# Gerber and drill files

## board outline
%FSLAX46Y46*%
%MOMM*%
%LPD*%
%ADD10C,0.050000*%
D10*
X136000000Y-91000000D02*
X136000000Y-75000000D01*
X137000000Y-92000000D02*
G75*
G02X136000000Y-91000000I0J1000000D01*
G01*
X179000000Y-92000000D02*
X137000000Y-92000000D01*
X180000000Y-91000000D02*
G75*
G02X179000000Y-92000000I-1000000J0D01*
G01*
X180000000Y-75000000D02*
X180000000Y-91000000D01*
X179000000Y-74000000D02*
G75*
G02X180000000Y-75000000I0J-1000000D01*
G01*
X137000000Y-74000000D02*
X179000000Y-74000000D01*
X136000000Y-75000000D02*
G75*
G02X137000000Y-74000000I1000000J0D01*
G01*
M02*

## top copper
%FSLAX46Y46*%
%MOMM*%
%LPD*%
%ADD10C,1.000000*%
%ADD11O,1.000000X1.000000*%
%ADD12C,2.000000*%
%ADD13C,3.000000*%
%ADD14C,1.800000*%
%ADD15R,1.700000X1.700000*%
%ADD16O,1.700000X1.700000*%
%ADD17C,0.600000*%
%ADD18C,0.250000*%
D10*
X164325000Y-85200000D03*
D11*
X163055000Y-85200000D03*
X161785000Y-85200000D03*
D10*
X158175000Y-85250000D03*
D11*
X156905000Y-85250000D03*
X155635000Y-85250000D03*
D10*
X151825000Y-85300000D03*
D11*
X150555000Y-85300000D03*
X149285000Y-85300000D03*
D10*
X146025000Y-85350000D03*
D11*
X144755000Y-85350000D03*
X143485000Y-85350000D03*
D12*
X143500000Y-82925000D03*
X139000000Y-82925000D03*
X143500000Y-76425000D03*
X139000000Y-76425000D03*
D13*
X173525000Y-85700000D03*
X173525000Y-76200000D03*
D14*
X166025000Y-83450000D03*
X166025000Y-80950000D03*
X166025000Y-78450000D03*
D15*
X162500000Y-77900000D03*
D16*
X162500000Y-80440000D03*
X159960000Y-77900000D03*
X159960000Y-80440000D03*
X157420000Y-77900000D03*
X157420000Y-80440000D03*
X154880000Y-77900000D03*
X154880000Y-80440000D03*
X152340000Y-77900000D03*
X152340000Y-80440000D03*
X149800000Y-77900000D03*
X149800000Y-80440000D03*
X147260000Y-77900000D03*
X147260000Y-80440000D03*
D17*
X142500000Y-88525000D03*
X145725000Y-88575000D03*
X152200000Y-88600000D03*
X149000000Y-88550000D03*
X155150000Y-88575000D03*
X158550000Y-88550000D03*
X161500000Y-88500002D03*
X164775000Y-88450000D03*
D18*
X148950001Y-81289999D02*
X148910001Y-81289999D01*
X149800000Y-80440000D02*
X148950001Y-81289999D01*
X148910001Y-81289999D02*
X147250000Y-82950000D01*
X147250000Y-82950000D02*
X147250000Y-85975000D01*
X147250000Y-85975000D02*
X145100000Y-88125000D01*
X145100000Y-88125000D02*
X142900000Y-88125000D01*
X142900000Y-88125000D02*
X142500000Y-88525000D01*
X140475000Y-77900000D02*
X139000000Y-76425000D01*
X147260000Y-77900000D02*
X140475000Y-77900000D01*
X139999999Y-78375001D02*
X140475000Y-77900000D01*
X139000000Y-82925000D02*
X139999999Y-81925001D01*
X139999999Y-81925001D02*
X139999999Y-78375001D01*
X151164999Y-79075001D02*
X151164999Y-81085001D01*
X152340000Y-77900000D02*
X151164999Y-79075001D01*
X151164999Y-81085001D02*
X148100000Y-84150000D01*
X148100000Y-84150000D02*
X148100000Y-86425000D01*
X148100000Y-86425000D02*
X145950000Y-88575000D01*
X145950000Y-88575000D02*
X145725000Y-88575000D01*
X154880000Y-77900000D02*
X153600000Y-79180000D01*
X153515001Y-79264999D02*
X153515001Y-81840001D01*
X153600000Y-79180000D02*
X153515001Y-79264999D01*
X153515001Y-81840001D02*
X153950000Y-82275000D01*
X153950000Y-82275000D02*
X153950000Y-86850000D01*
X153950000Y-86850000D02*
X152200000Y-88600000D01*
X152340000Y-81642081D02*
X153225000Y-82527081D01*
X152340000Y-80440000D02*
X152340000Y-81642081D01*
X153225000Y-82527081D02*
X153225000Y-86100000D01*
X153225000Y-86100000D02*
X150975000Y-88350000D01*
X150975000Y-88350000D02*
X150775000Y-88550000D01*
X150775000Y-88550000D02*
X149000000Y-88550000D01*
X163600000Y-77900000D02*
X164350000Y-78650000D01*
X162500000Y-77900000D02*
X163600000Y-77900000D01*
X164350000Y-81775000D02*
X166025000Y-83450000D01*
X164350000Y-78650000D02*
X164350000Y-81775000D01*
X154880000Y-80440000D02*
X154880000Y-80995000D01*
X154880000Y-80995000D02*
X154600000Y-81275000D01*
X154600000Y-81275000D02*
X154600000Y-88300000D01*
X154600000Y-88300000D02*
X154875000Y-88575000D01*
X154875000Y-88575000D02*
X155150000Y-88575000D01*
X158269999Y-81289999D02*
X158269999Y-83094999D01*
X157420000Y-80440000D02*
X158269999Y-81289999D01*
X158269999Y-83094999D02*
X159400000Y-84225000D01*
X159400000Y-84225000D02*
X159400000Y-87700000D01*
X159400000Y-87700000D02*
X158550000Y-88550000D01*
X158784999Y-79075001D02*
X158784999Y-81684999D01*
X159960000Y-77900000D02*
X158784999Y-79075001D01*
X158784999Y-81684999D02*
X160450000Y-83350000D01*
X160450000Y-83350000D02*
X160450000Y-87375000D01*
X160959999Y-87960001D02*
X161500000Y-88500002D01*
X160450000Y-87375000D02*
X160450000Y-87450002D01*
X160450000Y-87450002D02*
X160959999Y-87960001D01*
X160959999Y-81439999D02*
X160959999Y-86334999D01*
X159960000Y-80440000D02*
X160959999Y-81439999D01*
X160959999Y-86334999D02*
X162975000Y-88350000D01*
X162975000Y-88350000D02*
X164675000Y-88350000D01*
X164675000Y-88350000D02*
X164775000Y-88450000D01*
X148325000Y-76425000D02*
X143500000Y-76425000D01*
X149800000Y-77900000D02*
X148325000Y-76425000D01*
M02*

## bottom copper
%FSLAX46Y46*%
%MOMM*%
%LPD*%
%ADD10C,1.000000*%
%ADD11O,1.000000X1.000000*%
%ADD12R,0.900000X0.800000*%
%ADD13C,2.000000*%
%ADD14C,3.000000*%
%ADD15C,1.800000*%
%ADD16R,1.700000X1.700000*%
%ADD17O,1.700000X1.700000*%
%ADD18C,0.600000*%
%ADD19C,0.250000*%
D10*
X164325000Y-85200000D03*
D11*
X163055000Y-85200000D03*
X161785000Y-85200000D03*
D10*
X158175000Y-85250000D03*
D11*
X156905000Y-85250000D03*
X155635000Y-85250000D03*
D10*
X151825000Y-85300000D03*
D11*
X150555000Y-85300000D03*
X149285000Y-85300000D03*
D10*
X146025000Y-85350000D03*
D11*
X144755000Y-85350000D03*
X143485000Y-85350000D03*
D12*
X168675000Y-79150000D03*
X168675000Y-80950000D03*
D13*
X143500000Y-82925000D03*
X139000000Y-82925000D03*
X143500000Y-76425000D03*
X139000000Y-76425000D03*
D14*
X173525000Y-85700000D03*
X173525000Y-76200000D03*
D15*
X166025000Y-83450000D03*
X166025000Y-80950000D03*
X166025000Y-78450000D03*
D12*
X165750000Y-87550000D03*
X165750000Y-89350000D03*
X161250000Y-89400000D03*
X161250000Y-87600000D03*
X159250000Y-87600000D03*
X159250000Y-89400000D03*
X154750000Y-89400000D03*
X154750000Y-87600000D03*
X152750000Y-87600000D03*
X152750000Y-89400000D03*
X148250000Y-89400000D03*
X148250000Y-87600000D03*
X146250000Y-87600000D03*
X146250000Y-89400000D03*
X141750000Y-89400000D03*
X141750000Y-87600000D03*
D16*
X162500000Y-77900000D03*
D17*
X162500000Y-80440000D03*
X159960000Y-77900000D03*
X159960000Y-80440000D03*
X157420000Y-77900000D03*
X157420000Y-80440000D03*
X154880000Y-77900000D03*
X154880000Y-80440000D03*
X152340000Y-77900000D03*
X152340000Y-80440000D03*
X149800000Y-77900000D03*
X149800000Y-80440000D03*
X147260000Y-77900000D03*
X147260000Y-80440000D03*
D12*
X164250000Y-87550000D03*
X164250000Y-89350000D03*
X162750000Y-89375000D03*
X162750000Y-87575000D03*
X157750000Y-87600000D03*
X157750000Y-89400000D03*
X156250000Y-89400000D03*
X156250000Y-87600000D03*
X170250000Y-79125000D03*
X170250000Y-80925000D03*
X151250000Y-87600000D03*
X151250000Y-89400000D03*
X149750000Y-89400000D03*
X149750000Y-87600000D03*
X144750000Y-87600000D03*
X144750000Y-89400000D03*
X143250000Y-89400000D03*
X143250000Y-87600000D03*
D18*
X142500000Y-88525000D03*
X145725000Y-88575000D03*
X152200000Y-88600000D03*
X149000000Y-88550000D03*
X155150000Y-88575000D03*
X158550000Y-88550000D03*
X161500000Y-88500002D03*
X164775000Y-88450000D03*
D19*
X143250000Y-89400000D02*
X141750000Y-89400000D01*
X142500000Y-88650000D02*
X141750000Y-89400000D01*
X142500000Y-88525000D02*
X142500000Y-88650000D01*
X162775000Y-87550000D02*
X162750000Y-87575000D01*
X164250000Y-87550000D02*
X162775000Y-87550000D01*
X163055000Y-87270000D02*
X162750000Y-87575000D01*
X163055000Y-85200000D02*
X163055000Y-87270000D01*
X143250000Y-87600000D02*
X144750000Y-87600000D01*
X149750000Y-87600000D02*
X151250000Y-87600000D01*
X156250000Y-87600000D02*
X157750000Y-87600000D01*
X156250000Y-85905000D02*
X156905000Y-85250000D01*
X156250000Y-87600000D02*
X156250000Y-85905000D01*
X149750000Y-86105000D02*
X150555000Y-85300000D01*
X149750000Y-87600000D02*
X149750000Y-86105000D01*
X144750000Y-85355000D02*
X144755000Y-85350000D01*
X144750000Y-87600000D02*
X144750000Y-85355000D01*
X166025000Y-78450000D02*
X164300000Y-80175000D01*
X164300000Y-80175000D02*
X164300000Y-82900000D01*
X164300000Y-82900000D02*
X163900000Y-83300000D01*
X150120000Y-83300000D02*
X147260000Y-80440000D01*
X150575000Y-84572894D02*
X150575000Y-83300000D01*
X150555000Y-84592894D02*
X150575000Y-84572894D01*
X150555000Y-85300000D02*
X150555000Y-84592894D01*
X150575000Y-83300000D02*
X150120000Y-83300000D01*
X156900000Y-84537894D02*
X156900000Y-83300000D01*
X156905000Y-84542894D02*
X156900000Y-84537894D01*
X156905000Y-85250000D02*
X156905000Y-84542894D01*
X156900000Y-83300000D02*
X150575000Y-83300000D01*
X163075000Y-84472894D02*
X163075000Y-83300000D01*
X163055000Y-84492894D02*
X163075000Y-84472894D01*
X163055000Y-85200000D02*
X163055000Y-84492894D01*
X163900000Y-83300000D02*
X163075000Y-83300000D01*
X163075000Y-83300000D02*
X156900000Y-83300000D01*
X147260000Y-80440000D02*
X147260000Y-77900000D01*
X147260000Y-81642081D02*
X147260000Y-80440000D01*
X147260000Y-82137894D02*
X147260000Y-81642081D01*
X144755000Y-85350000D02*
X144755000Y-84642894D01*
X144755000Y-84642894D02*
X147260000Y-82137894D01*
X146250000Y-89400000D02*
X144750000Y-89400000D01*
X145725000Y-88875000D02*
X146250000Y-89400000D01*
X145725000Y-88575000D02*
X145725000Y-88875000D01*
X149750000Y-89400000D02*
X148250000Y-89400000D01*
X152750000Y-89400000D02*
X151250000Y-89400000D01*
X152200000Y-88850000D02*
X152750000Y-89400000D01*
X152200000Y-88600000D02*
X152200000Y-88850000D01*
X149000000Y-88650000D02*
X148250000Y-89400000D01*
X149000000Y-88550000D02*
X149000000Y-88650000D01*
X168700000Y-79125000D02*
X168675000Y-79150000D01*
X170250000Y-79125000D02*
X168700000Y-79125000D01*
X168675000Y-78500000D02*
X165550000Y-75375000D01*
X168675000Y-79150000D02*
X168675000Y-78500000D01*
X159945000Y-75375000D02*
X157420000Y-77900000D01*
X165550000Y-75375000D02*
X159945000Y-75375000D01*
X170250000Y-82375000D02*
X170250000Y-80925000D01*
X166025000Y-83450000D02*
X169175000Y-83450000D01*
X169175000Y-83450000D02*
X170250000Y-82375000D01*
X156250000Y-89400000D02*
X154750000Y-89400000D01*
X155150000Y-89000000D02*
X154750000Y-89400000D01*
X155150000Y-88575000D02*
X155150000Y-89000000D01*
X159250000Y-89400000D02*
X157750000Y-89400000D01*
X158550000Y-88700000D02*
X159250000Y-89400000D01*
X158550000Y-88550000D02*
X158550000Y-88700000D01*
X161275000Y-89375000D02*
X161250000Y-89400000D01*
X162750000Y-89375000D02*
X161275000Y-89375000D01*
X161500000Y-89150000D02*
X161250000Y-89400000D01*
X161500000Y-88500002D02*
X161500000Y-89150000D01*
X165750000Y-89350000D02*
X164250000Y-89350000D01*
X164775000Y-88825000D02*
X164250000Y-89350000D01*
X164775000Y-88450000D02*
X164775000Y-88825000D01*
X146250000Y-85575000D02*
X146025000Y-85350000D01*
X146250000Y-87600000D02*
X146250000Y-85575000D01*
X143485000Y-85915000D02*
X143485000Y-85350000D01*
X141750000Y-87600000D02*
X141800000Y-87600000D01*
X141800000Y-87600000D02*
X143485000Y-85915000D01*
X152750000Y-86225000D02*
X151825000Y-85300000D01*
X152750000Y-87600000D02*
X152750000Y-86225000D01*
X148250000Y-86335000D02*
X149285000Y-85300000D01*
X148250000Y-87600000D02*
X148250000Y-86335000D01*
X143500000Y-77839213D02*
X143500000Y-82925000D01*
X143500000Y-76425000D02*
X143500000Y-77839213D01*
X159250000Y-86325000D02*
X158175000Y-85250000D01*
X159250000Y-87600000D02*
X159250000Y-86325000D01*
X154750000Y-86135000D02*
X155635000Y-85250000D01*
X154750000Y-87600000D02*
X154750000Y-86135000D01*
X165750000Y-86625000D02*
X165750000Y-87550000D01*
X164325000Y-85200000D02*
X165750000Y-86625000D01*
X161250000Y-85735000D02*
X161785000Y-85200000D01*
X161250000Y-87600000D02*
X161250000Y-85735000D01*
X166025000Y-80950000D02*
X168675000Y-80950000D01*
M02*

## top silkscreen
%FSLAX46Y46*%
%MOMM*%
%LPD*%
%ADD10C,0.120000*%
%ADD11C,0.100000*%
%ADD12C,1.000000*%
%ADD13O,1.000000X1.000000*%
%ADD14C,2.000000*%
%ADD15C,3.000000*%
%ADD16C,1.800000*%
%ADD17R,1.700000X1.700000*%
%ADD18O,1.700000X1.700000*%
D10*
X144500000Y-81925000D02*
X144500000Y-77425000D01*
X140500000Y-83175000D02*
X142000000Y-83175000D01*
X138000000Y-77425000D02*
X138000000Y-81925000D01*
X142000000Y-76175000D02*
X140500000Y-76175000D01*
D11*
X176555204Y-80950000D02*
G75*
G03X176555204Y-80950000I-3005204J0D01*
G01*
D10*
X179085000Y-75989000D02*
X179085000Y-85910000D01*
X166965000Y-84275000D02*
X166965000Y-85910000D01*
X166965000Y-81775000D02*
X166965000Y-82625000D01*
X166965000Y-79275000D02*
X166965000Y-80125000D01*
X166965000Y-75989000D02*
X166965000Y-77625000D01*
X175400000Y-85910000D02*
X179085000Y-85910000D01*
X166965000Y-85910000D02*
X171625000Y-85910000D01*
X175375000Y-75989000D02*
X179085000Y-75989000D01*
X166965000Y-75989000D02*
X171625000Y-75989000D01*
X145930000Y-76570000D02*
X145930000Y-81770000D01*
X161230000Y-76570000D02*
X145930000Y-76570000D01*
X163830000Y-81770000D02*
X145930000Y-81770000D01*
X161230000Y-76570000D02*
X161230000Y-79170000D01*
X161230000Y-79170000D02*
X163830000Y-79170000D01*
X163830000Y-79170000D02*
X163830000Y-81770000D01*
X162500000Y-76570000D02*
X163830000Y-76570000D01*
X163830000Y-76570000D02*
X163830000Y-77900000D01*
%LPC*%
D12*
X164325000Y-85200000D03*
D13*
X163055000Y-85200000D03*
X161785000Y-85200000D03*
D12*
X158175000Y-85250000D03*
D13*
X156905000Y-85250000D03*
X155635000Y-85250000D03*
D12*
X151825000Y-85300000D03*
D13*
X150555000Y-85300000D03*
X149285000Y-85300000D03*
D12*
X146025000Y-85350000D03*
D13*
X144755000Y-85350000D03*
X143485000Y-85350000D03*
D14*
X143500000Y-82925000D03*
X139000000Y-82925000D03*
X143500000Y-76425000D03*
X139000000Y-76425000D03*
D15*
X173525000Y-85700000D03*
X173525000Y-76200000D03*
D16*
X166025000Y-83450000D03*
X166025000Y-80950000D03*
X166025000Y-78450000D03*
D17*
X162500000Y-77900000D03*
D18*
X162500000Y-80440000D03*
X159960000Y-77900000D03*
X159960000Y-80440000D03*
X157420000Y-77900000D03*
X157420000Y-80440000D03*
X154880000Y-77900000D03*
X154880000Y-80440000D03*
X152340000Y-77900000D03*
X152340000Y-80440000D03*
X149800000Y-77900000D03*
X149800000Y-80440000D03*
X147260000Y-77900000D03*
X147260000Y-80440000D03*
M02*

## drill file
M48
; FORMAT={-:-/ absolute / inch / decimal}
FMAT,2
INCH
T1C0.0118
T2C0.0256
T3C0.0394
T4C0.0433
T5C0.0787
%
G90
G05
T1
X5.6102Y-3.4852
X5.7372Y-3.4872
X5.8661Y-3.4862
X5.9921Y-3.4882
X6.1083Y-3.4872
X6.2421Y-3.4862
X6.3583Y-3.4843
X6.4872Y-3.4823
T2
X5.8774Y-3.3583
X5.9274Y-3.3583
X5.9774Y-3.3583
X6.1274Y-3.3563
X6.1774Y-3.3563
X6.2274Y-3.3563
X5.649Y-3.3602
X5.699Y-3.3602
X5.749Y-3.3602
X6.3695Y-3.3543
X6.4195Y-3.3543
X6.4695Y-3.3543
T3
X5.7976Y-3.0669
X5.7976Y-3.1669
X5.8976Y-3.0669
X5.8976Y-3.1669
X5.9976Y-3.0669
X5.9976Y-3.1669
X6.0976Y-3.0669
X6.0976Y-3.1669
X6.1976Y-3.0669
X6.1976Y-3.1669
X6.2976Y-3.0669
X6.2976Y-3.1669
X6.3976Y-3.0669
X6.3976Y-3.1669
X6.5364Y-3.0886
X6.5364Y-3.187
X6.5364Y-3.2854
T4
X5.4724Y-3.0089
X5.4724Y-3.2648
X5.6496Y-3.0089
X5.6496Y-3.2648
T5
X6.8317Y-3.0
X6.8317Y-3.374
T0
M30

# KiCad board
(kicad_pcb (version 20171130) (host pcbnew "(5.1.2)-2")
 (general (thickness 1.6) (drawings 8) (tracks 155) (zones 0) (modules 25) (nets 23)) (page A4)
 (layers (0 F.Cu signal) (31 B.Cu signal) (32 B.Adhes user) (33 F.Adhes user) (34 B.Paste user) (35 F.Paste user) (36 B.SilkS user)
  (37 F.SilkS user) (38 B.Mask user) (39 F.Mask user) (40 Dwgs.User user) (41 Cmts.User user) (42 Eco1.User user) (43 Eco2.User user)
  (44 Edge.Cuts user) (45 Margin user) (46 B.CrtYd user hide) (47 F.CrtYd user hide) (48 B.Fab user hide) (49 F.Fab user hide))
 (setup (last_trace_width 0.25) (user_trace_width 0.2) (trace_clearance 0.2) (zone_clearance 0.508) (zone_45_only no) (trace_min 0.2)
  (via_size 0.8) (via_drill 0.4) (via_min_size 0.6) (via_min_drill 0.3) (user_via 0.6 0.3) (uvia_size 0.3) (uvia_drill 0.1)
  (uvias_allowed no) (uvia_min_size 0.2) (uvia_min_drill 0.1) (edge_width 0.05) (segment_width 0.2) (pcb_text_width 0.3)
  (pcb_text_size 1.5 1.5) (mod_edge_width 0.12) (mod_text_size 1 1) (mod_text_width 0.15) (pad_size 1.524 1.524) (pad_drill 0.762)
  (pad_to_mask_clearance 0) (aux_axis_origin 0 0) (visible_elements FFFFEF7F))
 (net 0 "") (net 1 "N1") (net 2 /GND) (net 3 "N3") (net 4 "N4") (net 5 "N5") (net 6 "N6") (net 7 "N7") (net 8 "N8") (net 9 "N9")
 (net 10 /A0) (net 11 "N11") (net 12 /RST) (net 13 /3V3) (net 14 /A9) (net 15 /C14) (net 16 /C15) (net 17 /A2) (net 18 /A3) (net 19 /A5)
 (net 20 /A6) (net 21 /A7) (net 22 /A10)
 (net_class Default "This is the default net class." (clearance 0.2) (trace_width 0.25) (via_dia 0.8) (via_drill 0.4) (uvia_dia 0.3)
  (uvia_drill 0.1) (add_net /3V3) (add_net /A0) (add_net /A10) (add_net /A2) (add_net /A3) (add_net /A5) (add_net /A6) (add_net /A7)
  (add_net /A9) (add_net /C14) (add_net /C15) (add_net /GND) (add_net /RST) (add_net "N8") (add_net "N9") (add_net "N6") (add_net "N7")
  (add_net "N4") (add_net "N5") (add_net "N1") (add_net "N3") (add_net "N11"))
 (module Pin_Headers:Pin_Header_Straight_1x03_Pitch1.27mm (layer F.Cu) (at 164.325 85.2 270)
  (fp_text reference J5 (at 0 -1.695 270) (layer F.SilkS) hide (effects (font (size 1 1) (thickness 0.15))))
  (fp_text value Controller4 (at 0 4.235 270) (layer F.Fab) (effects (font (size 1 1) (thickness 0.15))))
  (pad 1 thru_hole circle (at 0 0 270) (size 1 1) (drill 0.65) (layers *.Cu *.Mask) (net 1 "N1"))
  (pad 2 thru_hole oval (at 0 1.27 270) (size 1 1) (drill 0.65) (layers *.Cu *.Mask) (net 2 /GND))
  (pad 3 thru_hole oval (at 0 2.54 270) (size 1 1) (drill 0.65) (layers *.Cu *.Mask) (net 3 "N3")))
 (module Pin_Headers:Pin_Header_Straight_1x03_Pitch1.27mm (layer F.Cu) (at 158.175 85.25 270)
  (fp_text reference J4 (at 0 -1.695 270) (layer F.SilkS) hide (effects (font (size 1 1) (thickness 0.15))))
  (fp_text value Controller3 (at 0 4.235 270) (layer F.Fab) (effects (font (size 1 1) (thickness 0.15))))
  (pad 1 thru_hole circle (at 0 0 270) (size 1 1) (drill 0.65) (layers *.Cu *.Mask) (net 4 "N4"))
  (pad 2 thru_hole oval (at 0 1.27 270) (size 1 1) (drill 0.65) (layers *.Cu *.Mask) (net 2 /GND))
  (pad 3 thru_hole oval (at 0 2.54 270) (size 1 1) (drill 0.65) (layers *.Cu *.Mask) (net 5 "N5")))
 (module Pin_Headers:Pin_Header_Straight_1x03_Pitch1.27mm (layer F.Cu) (at 151.825 85.3 270)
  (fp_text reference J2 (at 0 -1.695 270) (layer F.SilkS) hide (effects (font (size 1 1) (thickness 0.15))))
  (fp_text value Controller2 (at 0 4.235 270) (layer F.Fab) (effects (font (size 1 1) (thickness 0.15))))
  (pad 1 thru_hole circle (at 0 0 270) (size 1 1) (drill 0.65) (layers *.Cu *.Mask) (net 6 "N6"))
  (pad 2 thru_hole oval (at 0 1.27 270) (size 1 1) (drill 0.65) (layers *.Cu *.Mask) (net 2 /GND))
  (pad 3 thru_hole oval (at 0 2.54 270) (size 1 1) (drill 0.65) (layers *.Cu *.Mask) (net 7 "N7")))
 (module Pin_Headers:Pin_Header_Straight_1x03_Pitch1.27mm (layer F.Cu) (at 146.025 85.35 270)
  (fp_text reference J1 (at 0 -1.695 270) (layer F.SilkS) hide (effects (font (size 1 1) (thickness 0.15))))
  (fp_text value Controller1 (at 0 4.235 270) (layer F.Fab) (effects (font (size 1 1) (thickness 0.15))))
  (pad 1 thru_hole circle (at 0 0 270) (size 1 1) (drill 0.65) (layers *.Cu *.Mask) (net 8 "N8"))
  (pad 2 thru_hole oval (at 0 1.27 270) (size 1 1) (drill 0.65) (layers *.Cu *.Mask) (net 2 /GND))
  (pad 3 thru_hole oval (at 0 2.54 270) (size 1 1) (drill 0.65) (layers *.Cu *.Mask) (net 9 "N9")))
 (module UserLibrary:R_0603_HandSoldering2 (layer B.Cu) (at 168.675 80.05 90)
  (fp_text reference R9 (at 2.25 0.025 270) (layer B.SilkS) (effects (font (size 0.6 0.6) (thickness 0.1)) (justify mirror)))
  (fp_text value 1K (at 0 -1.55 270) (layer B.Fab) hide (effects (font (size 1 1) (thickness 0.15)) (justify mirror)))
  (pad 2 smd rect (at 0.9 0 90) (size 0.8 0.9) (layers B.Cu B.Paste B.Mask) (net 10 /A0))
  (pad 1 smd rect (at -0.9 0 90) (size 0.8 0.9) (layers B.Cu B.Paste B.Mask) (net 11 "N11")))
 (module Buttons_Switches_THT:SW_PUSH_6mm (layer F.Cu) (at 139 82.925 90)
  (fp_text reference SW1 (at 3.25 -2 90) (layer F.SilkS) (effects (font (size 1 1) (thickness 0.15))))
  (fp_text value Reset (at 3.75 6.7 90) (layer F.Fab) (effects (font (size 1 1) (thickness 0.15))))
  (fp_line (start 1 5.5) (end 5.5 5.5) (layer F.SilkS) (width 0.12))
  (fp_line (start -0.25 1.5) (end -0.25 3) (layer F.SilkS) (width 0.12))
  (fp_line (start 5.5 -1) (end 1 -1) (layer F.SilkS) (width 0.12))
  (fp_line (start 6.75 3) (end 6.75 1.5) (layer F.SilkS) (width 0.12))
  (pad 2 thru_hole circle (at 0 4.5 180) (size 2 2) (drill 1.1) (layers *.Cu *.Mask) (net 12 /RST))
  (pad 1 thru_hole circle (at 0 0 180) (size 2 2) (drill 1.1) (layers *.Cu *.Mask) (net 2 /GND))
  (pad 2 thru_hole circle (at 6.5 4.5 180) (size 2 2) (drill 1.1) (layers *.Cu *.Mask) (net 12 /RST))
  (pad 1 thru_hole circle (at 6.5 0 180) (size 2 2) (drill 1.1) (layers *.Cu *.Mask) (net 2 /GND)))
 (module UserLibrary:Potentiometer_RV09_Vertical (layer F.Cu) (at 173.525 80.95)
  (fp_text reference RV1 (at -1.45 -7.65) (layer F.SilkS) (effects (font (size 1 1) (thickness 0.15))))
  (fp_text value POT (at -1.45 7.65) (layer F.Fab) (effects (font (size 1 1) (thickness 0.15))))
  (fp_circle (center 0.025 0) (end 2.45 1.775) (layer F.SilkS) (width 0.1))
  (fp_line (start 5.56 -4.961) (end 5.56 4.96) (layer F.SilkS) (width 0.12))
  (fp_line (start -6.56 3.325) (end -6.56 4.96) (layer F.SilkS) (width 0.12))
  (fp_line (start -6.56 0.825) (end -6.56 1.675) (layer F.SilkS) (width 0.12))
  (fp_line (start -6.56 -1.675) (end -6.56 -0.825) (layer F.SilkS) (width 0.12))
  (fp_line (start -6.56 -4.961) (end -6.56 -3.325) (layer F.SilkS) (width 0.12))
  (fp_line (start 1.875 4.96) (end 5.56 4.96) (layer F.SilkS) (width 0.12))
  (fp_line (start -6.56 4.96) (end -1.9 4.96) (layer F.SilkS) (width 0.12))
  (fp_line (start 1.85 -4.961) (end 5.56 -4.961) (layer F.SilkS) (width 0.12))
  (fp_line (start -6.56 -4.961) (end -1.9 -4.961) (layer F.SilkS) (width 0.12))
  (pad "" thru_hole circle (at 0 4.75) (size 3 3) (drill 2) (layers *.Cu *.Mask))
  (pad "" thru_hole circle (at 0 -4.75) (size 3 3) (drill 2) (layers *.Cu *.Mask))
  (pad 1 thru_hole circle (at -7.5 2.5) (size 1.8 1.8) (drill 1) (layers *.Cu *.Mask) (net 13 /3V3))
  (pad 2 thru_hole circle (at -7.5 0) (size 1.8 1.8) (drill 1) (layers *.Cu *.Mask) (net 11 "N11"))
  (pad 3 thru_hole circle (at -7.5 -2.5) (size 1.8 1.8) (drill 1) (layers *.Cu *.Mask) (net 2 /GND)))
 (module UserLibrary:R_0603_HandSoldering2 (layer B.Cu) (at 165.75 88.45 90)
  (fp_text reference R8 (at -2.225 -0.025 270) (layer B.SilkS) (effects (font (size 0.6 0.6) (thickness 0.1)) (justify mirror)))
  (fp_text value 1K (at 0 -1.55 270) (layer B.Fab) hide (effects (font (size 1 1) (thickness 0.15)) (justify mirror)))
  (pad 2 smd rect (at 0.9 0 90) (size 0.8 0.9) (layers B.Cu B.Paste B.Mask) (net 1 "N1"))
  (pad 1 smd rect (at -0.9 0 90) (size 0.8 0.9) (layers B.Cu B.Paste B.Mask) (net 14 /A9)))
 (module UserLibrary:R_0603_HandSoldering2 (layer B.Cu) (at 161.25 88.5 270)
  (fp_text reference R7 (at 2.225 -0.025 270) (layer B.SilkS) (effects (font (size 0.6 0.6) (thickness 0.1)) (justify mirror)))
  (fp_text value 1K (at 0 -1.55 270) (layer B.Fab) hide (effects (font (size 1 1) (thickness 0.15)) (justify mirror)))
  (pad 2 smd rect (at 0.9 0 270) (size 0.8 0.9) (layers B.Cu B.Paste B.Mask) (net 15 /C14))
  (pad 1 smd rect (at -0.9 0 270) (size 0.8 0.9) (layers B.Cu B.Paste B.Mask) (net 3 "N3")))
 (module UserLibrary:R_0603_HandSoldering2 (layer B.Cu) (at 159.25 88.5 90)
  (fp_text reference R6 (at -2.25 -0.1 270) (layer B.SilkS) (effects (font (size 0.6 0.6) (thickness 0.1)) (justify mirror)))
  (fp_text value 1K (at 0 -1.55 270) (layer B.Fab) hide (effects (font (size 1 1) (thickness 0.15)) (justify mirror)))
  (pad 2 smd rect (at 0.9 0 90) (size 0.8 0.9) (layers B.Cu B.Paste B.Mask) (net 4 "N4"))
  (pad 1 smd rect (at -0.9 0 90) (size 0.8 0.9) (layers B.Cu B.Paste B.Mask) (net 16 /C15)))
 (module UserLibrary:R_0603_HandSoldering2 (layer B.Cu) (at 154.75 88.5 270)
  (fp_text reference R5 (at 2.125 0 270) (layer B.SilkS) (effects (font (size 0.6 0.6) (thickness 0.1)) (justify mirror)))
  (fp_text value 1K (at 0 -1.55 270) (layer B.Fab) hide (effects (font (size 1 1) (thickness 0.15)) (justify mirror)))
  (pad 2 smd rect (at 0.9 0 270) (size 0.8 0.9) (layers B.Cu B.Paste B.Mask) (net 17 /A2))
  (pad 1 smd rect (at -0.9 0 270) (size 0.8 0.9) (layers B.Cu B.Paste B.Mask) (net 5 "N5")))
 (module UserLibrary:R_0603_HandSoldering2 (layer B.Cu) (at 152.75 88.5 90)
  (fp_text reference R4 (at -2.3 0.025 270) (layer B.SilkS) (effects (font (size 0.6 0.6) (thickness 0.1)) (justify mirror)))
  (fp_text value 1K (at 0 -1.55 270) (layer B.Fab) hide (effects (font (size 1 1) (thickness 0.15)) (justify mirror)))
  (pad 2 smd rect (at 0.9 0 90) (size 0.8 0.9) (layers B.Cu B.Paste B.Mask) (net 6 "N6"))
  (pad 1 smd rect (at -0.9 0 90) (size 0.8 0.9) (layers B.Cu B.Paste B.Mask) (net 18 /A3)))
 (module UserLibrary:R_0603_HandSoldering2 (layer B.Cu) (at 148.25 88.5 270)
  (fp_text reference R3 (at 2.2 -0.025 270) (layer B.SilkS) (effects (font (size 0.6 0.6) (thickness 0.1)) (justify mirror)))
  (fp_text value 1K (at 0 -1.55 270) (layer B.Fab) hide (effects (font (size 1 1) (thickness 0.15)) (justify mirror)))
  (pad 2 smd rect (at 0.9 0 270) (size 0.8 0.9) (layers B.Cu B.Paste B.Mask) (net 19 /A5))
  (pad 1 smd rect (at -0.9 0 270) (size 0.8 0.9) (layers B.Cu B.Paste B.Mask) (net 7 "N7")))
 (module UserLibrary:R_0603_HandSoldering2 (layer B.Cu) (at 146.25 88.5 90)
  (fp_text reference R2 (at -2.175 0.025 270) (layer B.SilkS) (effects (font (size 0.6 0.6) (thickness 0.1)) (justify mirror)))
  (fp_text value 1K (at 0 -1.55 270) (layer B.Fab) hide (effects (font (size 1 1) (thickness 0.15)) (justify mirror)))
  (pad 2 smd rect (at 0.9 0 90) (size 0.8 0.9) (layers B.Cu B.Paste B.Mask) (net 8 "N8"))
  (pad 1 smd rect (at -0.9 0 90) (size 0.8 0.9) (layers B.Cu B.Paste B.Mask) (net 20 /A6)))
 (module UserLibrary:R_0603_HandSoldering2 (layer B.Cu) (at 141.75 88.5 270)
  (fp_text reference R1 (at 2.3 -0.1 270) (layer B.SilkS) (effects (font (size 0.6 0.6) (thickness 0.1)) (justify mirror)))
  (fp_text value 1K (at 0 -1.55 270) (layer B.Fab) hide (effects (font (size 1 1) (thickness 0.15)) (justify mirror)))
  (pad 2 smd rect (at 0.9 0 270) (size 0.8 0.9) (layers B.Cu B.Paste B.Mask) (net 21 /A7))
  (pad 1 smd rect (at -0.9 0 270) (size 0.8 0.9) (layers B.Cu B.Paste B.Mask) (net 9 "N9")))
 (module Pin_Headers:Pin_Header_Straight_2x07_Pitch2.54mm (layer F.Cu) (at 162.5 77.9 270)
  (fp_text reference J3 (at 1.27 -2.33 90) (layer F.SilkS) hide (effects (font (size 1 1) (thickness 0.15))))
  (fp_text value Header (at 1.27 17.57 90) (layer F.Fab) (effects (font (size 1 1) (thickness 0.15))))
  (fp_line (start -1.33 16.57) (end 3.87 16.57) (layer F.SilkS) (width 0.12))
  (fp_line (start -1.33 1.27) (end -1.33 16.57) (layer F.SilkS) (width 0.12))
  (fp_line (start 3.87 -1.33) (end 3.87 16.57) (layer F.SilkS) (width 0.12))
  (fp_line (start -1.33 1.27) (end 1.27 1.27) (layer F.SilkS) (width 0.12))
  (fp_line (start 1.27 1.27) (end 1.27 -1.33) (layer F.SilkS) (width 0.12))
  (fp_line (start 1.27 -1.33) (end 3.87 -1.33) (layer F.SilkS) (width 0.12))
  (fp_line (start -1.33 0) (end -1.33 -1.33) (layer F.SilkS) (width 0.12))
  (fp_line (start -1.33 -1.33) (end 0 -1.33) (layer F.SilkS) (width 0.12))
  (pad 1 thru_hole rect (at 0 0 270) (size 1.7 1.7) (drill 1) (layers *.Cu *.Mask) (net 13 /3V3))
  (pad 2 thru_hole oval (at 2.54 0 270) (size 1.7 1.7) (drill 1) (layers *.Cu *.Mask) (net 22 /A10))
  (pad 3 thru_hole oval (at 0 2.54 270) (size 1.7 1.7) (drill 1) (layers *.Cu *.Mask) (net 15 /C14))
  (pad 4 thru_hole oval (at 2.54 2.54 270) (size 1.7 1.7) (drill 1) (layers *.Cu *.Mask) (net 14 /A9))
  (pad 5 thru_hole oval (at 0 5.08 270) (size 1.7 1.7) (drill 1) (layers *.Cu *.Mask) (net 10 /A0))
  (pad 6 thru_hole oval (at 2.54 5.08 270) (size 1.7 1.7) (drill 1) (layers *.Cu *.Mask) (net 16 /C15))
  (pad 7 thru_hole oval (at 0 7.62 270) (size 1.7 1.7) (drill 1) (layers *.Cu *.Mask) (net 18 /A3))
  (pad 8 thru_hole oval (at 2.54 7.62 270) (size 1.7 1.7) (drill 1) (layers *.Cu *.Mask) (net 17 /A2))
  (pad 9 thru_hole oval (at 0 10.16 270) (size 1.7 1.7) (drill 1) (layers *.Cu *.Mask) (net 20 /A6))
  (pad 10 thru_hole oval (at 2.54 10.16 270) (size 1.7 1.7) (drill 1) (layers *.Cu *.Mask) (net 19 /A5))
  (pad 11 thru_hole oval (at 0 12.7 270) (size 1.7 1.7) (drill 1) (layers *.Cu *.Mask) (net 12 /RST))
  (pad 12 thru_hole oval (at 2.54 12.7 270) (size 1.7 1.7) (drill 1) (layers *.Cu *.Mask) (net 21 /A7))
  (pad 13 thru_hole oval (at 0 15.24 270) (size 1.7 1.7) (drill 1) (layers *.Cu *.Mask) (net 2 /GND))
  (pad 14 thru_hole oval (at 2.54 15.24 270) (size 1.7 1.7) (drill 1) (layers *.Cu *.Mask) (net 2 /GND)))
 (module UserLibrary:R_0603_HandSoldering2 (layer B.Cu) (at 164.25 88.45 90)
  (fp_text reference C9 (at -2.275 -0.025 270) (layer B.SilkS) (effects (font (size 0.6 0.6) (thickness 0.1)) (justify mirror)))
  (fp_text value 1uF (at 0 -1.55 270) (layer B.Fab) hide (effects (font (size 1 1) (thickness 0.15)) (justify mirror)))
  (pad 2 smd rect (at 0.9 0 90) (size 0.8 0.9) (layers B.Cu B.Paste B.Mask) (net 2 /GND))
  (pad 1 smd rect (at -0.9 0 90) (size 0.8 0.9) (layers B.Cu B.Paste B.Mask) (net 14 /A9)))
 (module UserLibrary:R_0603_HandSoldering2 (layer B.Cu) (at 162.75 88.475 270)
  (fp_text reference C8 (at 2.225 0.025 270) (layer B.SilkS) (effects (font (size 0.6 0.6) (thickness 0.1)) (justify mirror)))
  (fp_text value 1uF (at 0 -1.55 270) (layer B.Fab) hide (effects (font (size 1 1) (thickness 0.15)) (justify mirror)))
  (pad 2 smd rect (at 0.9 0 270) (size 0.8 0.9) (layers B.Cu B.Paste B.Mask) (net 15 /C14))
  (pad 1 smd rect (at -0.9 0 270) (size 0.8 0.9) (layers B.Cu B.Paste B.Mask) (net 2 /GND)))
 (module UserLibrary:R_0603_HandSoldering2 (layer B.Cu) (at 157.75 88.5 90)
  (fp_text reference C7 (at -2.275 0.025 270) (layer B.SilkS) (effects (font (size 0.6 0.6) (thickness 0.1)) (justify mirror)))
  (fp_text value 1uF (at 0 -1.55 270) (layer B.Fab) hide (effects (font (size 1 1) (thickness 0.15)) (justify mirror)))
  (pad 2 smd rect (at 0.9 0 90) (size 0.8 0.9) (layers B.Cu B.Paste B.Mask) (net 2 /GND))
  (pad 1 smd rect (at -0.9 0 90) (size 0.8 0.9) (layers B.Cu B.Paste B.Mask) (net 16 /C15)))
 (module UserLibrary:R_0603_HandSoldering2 (layer B.Cu) (at 156.25 88.5 270)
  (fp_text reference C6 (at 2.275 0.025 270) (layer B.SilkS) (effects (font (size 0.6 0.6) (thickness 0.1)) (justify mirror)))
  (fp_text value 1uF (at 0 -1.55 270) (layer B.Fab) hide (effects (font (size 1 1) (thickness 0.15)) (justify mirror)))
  (pad 2 smd rect (at 0.9 0 270) (size 0.8 0.9) (layers B.Cu B.Paste B.Mask) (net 17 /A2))
  (pad 1 smd rect (at -0.9 0 270) (size 0.8 0.9) (layers B.Cu B.Paste B.Mask) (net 2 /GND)))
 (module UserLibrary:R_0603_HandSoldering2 (layer B.Cu) (at 170.25 80.025 90)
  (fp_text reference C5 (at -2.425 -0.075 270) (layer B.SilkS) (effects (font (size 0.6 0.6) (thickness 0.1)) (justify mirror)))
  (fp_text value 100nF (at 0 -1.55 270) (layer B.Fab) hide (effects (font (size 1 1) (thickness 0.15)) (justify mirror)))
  (pad 2 smd rect (at 0.9 0 90) (size 0.8 0.9) (layers B.Cu B.Paste B.Mask) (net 10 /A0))
  (pad 1 smd rect (at -0.9 0 90) (size 0.8 0.9) (layers B.Cu B.Paste B.Mask) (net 13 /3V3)))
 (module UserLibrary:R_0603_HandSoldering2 (layer B.Cu) (at 151.25 88.5 90)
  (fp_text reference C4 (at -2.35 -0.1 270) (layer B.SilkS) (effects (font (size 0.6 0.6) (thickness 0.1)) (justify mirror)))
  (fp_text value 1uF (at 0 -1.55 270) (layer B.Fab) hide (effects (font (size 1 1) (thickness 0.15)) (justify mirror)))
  (pad 2 smd rect (at 0.9 0 90) (size 0.8 0.9) (layers B.Cu B.Paste B.Mask) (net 2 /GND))
  (pad 1 smd rect (at -0.9 0 90) (size 0.8 0.9) (layers B.Cu B.Paste B.Mask) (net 18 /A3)))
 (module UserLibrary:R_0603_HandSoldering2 (layer B.Cu) (at 149.75 88.5 270)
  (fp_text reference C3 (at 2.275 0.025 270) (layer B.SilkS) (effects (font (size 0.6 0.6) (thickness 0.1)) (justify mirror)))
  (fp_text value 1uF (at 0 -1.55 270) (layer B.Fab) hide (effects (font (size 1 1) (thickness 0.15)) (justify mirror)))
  (pad 2 smd rect (at 0.9 0 270) (size 0.8 0.9) (layers B.Cu B.Paste B.Mask) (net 19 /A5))
  (pad 1 smd rect (at -0.9 0 270) (size 0.8 0.9) (layers B.Cu B.Paste B.Mask) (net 2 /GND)))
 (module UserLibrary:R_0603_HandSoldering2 (layer B.Cu) (at 144.75 88.5 90)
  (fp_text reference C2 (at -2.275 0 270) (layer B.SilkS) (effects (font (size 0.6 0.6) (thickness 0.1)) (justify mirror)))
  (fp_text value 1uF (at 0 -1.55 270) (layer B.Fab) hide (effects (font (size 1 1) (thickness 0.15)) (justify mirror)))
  (pad 2 smd rect (at 0.9 0 90) (size 0.8 0.9) (layers B.Cu B.Paste B.Mask) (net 2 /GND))
  (pad 1 smd rect (at -0.9 0 90) (size 0.8 0.9) (layers B.Cu B.Paste B.Mask) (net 20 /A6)))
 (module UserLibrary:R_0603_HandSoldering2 (layer B.Cu) (at 143.25 88.5 270)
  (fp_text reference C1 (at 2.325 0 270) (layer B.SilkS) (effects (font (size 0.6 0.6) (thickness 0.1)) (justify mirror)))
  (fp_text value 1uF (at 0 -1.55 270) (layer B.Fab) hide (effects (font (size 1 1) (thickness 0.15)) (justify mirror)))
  (pad 2 smd rect (at 0.9 0 270) (size 0.8 0.9) (layers B.Cu B.Paste B.Mask) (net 21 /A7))
  (pad 1 smd rect (at -0.9 0 270) (size 0.8 0.9) (layers B.Cu B.Paste B.Mask) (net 2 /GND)))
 (gr_line (start 136 91) (end 136 75) (layer Edge.Cuts) (width 0.05))
 (gr_arc (start 137 91) (end 136 91) (angle -90) (layer Edge.Cuts) (width 0.05))
 (gr_line (start 179 92) (end 137 92) (layer Edge.Cuts) (width 0.05))
 (gr_arc (start 179 91) (end 179 92) (angle -90) (layer Edge.Cuts) (width 0.05))
 (gr_line (start 180 75) (end 180 91) (layer Edge.Cuts) (width 0.05))
 (gr_arc (start 179 75) (end 180 75) (angle -90) (layer Edge.Cuts) (width 0.05))
 (gr_line (start 137 74) (end 179 74) (layer Edge.Cuts) (width 0.05))
 (gr_arc (start 137 75) (end 137 74) (angle -90) (layer Edge.Cuts) (width 0.05))
 (segment (start 143.25 89.4) (end 141.75 89.4) (width 0.25) (layer B.Cu) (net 21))
 (segment (start 148.950001 81.289999) (end 148.910001 81.289999) (width 0.25) (layer F.Cu) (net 21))
 (segment (start 149.8 80.44) (end 148.950001 81.289999) (width 0.25) (layer F.Cu) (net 21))
 (segment (start 148.910001 81.289999) (end 147.25 82.95) (width 0.25) (layer F.Cu) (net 21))
 (segment (start 147.25 82.95) (end 147.25 85.975) (width 0.25) (layer F.Cu) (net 21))
 (segment (start 147.25 85.975) (end 145.1 88.125) (width 0.25) (layer F.Cu) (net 21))
 (via (at 142.5 88.525) (size 0.6) (drill 0.3) (layers F.Cu B.Cu) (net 21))
 (segment (start 145.1 88.125) (end 142.9 88.125) (width 0.25) (layer F.Cu) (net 21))
 (segment (start 142.9 88.125) (end 142.5 88.525) (width 0.25) (layer F.Cu) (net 21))
 (segment (start 142.5 88.65) (end 141.75 89.4) (width 0.25) (layer B.Cu) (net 21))
 (segment (start 142.5 88.525) (end 142.5 88.65) (width 0.25) (layer B.Cu) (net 21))
 (segment (start 140.475 77.9) (end 139 76.425) (width 0.25) (layer F.Cu) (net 2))
 (segment (start 147.26 77.9) (end 140.475 77.9) (width 0.25) (layer F.Cu) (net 2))
 (segment (start 139.999999 78.375001) (end 140.475 77.9) (width 0.25) (layer F.Cu) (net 2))
 (segment (start 139 82.925) (end 139.999999 81.925001) (width 0.25) (layer F.Cu) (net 2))
 (segment (start 139.999999 81.925001) (end 139.999999 78.375001) (width 0.25) (layer F.Cu) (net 2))
 (segment (start 162.775 87.55) (end 162.75 87.575) (width 0.25) (layer B.Cu) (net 2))
 (segment (start 164.25 87.55) (end 162.775 87.55) (width 0.25) (layer B.Cu) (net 2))
 (segment (start 163.055 87.27) (end 162.75 87.575) (width 0.25) (layer B.Cu) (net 2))
 (segment (start 163.055 85.2) (end 163.055 87.27) (width 0.25) (layer B.Cu) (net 2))
 (segment (start 143.25 87.6) (end 144.75 87.6) (width 0.25) (layer B.Cu) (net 2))
 (segment (start 149.75 87.6) (end 151.25 87.6) (width 0.25) (layer B.Cu) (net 2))
 (segment (start 156.25 87.6) (end 157.75 87.6) (width 0.25) (layer B.Cu) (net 2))
 (segment (start 156.25 85.905) (end 156.905 85.25) (width 0.25) (layer B.Cu) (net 2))
 (segment (start 156.25 87.6) (end 156.25 85.905) (width 0.25) (layer B.Cu) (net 2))
 (segment (start 149.75 86.105) (end 150.555 85.3) (width 0.25) (layer B.Cu) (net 2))
 (segment (start 149.75 87.6) (end 149.75 86.105) (width 0.25) (layer B.Cu) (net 2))
 (segment (start 144.75 85.355) (end 144.755 85.35) (width 0.25) (layer B.Cu) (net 2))
 (segment (start 144.75 87.6) (end 144.75 85.355) (width 0.25) (layer B.Cu) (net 2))
 (segment (start 166.025 78.45) (end 164.3 80.175) (width 0.25) (layer B.Cu) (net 2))
 (segment (start 164.3 80.175) (end 164.3 82.9) (width 0.25) (layer B.Cu) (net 2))
 (segment (start 164.3 82.9) (end 163.9 83.3) (width 0.25) (layer B.Cu) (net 2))
 (segment (start 150.12 83.3) (end 147.26 80.44) (width 0.25) (layer B.Cu) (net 2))
 (segment (start 150.575 84.572894) (end 150.575 83.3) (width 0.25) (layer B.Cu) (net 2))
 (segment (start 150.555 84.592894) (end 150.575 84.572894) (width 0.25) (layer B.Cu) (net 2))
 (segment (start 150.555 85.3) (end 150.555 84.592894) (width 0.25) (layer B.Cu) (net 2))
 (segment (start 150.575 83.3) (end 150.12 83.3) (width 0.25) (layer B.Cu) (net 2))
 (segment (start 156.9 84.537894) (end 156.9 83.3) (width 0.25) (layer B.Cu) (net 2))
 (segment (start 156.905 84.542894) (end 156.9 84.537894) (width 0.25) (layer B.Cu) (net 2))
 (segment (start 156.905 85.25) (end 156.905 84.542894) (width 0.25) (layer B.Cu) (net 2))
 (segment (start 156.9 83.3) (end 150.575 83.3) (width 0.25) (layer B.Cu) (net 2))
 (segment (start 163.075 84.472894) (end 163.075 83.3) (width 0.25) (layer B.Cu) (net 2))
 (segment (start 163.055 84.492894) (end 163.075 84.472894) (width 0.25) (layer B.Cu) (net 2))
 (segment (start 163.055 85.2) (end 163.055 84.492894) (width 0.25) (layer B.Cu) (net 2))
 (segment (start 163.9 83.3) (end 163.075 83.3) (width 0.25) (layer B.Cu) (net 2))
 (segment (start 163.075 83.3) (end 156.9 83.3) (width 0.25) (layer B.Cu) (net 2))
 (segment (start 147.26 80.44) (end 147.26 77.9) (width 0.25) (layer B.Cu) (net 2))
 (segment (start 147.26 81.642081) (end 147.26 80.44) (width 0.25) (layer B.Cu) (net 2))
 (segment (start 147.26 82.137894) (end 147.26 81.642081) (width 0.25) (layer B.Cu) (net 2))
 (segment (start 144.755 85.35) (end 144.755 84.642894) (width 0.25) (layer B.Cu) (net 2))
 (segment (start 144.755 84.642894) (end 147.26 82.137894) (width 0.25) (layer B.Cu) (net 2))
 (segment (start 146.25 89.4) (end 144.75 89.4) (width 0.25) (layer B.Cu) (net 20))
 (segment (start 151.164999 79.075001) (end 151.164999 81.085001) (width 0.25) (layer F.Cu) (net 20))
 (segment (start 152.34 77.9) (end 151.164999 79.075001) (width 0.25) (layer F.Cu) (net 20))
 (segment (start 151.164999 81.085001) (end 148.1 84.15) (width 0.25) (layer F.Cu) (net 20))
 (segment (start 148.1 84.15) (end 148.1 86.425) (width 0.25) (layer F.Cu) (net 20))
 (via (at 145.725 88.575) (size 0.6) (drill 0.3) (layers F.Cu B.Cu) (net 20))
 (segment (start 148.1 86.425) (end 145.95 88.575) (width 0.25) (layer F.Cu) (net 20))
 (segment (start 145.95 88.575) (end 145.725 88.575) (width 0.25) (layer F.Cu) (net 20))
 (segment (start 145.725 88.875) (end 146.25 89.4) (width 0.25) (layer B.Cu) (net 20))
 (segment (start 145.725 88.575) (end 145.725 88.875) (width 0.25) (layer B.Cu) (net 20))
 (segment (start 149.75 89.4) (end 148.25 89.4) (width 0.25) (layer B.Cu) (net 19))
 (segment (start 152.75 89.4) (end 151.25 89.4) (width 0.25) (layer B.Cu) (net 18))
 (segment (start 154.88 77.9) (end 153.6 79.18) (width 0.25) (layer F.Cu) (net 18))
 (segment (start 153.515001 79.264999) (end 153.515001 81.840001) (width 0.25) (layer F.Cu) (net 18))
 (segment (start 153.6 79.18) (end 153.515001 79.264999) (width 0.25) (layer F.Cu) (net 18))
 (segment (start 153.515001 81.840001) (end 153.95 82.275) (width 0.25) (layer F.Cu) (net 18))
 (via (at 152.2 88.6) (size 0.6) (drill 0.3) (layers F.Cu B.Cu) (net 18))
 (segment (start 153.95 82.275) (end 153.95 86.85) (width 0.25) (layer F.Cu) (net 18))
 (segment (start 153.95 86.85) (end 152.2 88.6) (width 0.25) (layer F.Cu) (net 18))
 (segment (start 152.2 88.85) (end 152.75 89.4) (width 0.25) (layer B.Cu) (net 18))
 (segment (start 152.2 88.6) (end 152.2 88.85) (width 0.25) (layer B.Cu) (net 18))
 (segment (start 152.34 81.642081) (end 153.225 82.527081) (width 0.25) (layer F.Cu) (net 19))
 (segment (start 152.34 80.44) (end 152.34 81.642081) (width 0.25) (layer F.Cu) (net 19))
 (segment (start 153.225 82.527081) (end 153.225 86.1) (width 0.25) (layer F.Cu) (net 19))
 (segment (start 153.225 86.1) (end 150.975 88.35) (width 0.25) (layer F.Cu) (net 19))
 (via (at 149 88.55) (size 0.6) (drill 0.3) (layers F.Cu B.Cu) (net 19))
 (segment (start 150.975 88.35) (end 150.775 88.55) (width 0.25) (layer F.Cu) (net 19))
 (segment (start 150.775 88.55) (end 149 88.55) (width 0.25) (layer F.Cu) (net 19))
 (segment (start 149 88.65) (end 148.25 89.4) (width 0.25) (layer B.Cu) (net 19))
 (segment (start 149 88.55) (end 149 88.65) (width 0.25) (layer B.Cu) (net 19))
 (segment (start 168.7 79.125) (end 168.675 79.15) (width 0.25) (layer B.Cu) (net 10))
 (segment (start 170.25 79.125) (end 168.7 79.125) (width 0.25) (layer B.Cu) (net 10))
 (segment (start 168.675 78.5) (end 165.55 75.375) (width 0.25) (layer B.Cu) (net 10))
 (segment (start 168.675 79.15) (end 168.675 78.5) (width 0.25) (layer B.Cu) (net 10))
 (segment (start 159.945 75.375) (end 157.42 77.9) (width 0.25) (layer B.Cu) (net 10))
 (segment (start 165.55 75.375) (end 159.945 75.375) (width 0.25) (layer B.Cu) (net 10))
 (segment (start 163.6 77.9) (end 164.35 78.65) (width 0.25) (layer F.Cu) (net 13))
 (segment (start 162.5 77.9) (end 163.6 77.9) (width 0.25) (layer F.Cu) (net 13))
 (segment (start 164.35 81.775) (end 166.025 83.45) (width 0.25) (layer F.Cu) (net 13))
 (segment (start 164.35 78.65) (end 164.35 81.775) (width 0.25) (layer F.Cu) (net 13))
 (segment (start 170.25 82.375) (end 170.25 80.925) (width 0.25) (layer B.Cu) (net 13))
 (segment (start 166.025 83.45) (end 169.175 83.45) (width 0.25) (layer B.Cu) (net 13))
 (segment (start 169.175 83.45) (end 170.25 82.375) (width 0.25) (layer B.Cu) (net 13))
 (segment (start 156.25 89.4) (end 154.75 89.4) (width 0.25) (layer B.Cu) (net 17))
 (segment (start 154.88 80.44) (end 154.88 80.995) (width 0.25) (layer F.Cu) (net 17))
 (segment (start 154.88 80.995) (end 154.6 81.275) (width 0.25) (layer F.Cu) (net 17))
 (segment (start 154.6 81.275) (end 154.6 88.3) (width 0.25) (layer F.Cu) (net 17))
 (via (at 155.15 88.575) (size 0.6) (drill 0.3) (layers F.Cu B.Cu) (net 17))
 (segment (start 154.6 88.3) (end 154.875 88.575) (width 0.25) (layer F.Cu) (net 17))
 (segment (start 154.875 88.575) (end 155.15 88.575) (width 0.25) (layer F.Cu) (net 17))
 (segment (start 155.15 89) (end 154.75 89.4) (width 0.25) (layer B.Cu) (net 17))
 (segment (start 155.15 88.575) (end 155.15 89) (width 0.25) (layer B.Cu) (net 17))
 (segment (start 159.25 89.4) (end 157.75 89.4) (width 0.25) (layer B.Cu) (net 16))
 (segment (start 158.269999 81.289999) (end 158.269999 83.094999) (width 0.25) (layer F.Cu) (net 16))
 (segment (start 157.42 80.44) (end 158.269999 81.289999) (width 0.25) (layer F.Cu) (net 16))
 (segment (start 158.269999 83.094999) (end 159.4 84.225) (width 0.25) (layer F.Cu) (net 16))
 (via (at 158.55 88.55) (size 0.6) (drill 0.3) (layers F.Cu B.Cu) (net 16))
 (segment (start 159.4 84.225) (end 159.4 87.7) (width 0.25) (layer F.Cu) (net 16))
 (segment (start 159.4 87.7) (end 158.55 88.55) (width 0.25) (layer F.Cu) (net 16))
 (segment (start 158.55 88.7) (end 159.25 89.4) (width 0.25) (layer B.Cu) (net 16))
 (segment (start 158.55 88.55) (end 158.55 88.7) (width 0.25) (layer B.Cu) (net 16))
 (segment (start 161.275 89.375) (end 161.25 89.4) (width 0.25) (layer B.Cu) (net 15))
 (segment (start 162.75 89.375) (end 161.275 89.375) (width 0.25) (layer B.Cu) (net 15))
 (segment (start 158.784999 79.075001) (end 158.784999 81.684999) (width 0.25) (layer F.Cu) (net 15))
 (segment (start 159.96 77.9) (end 158.784999 79.075001) (width 0.25) (layer F.Cu) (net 15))
 (segment (start 158.784999 81.684999) (end 160.45 83.35) (width 0.25) (layer F.Cu) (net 15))
 (segment (start 160.45 83.35) (end 160.45 87.375) (width 0.25) (layer F.Cu) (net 15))
 (via (at 161.5 88.500002) (size 0.6) (drill 0.3) (layers F.Cu B.Cu) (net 15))
 (segment (start 160.959999 87.960001) (end 161.5 88.500002) (width 0.25) (layer F.Cu) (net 15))
 (segment (start 160.45 87.375) (end 160.45 87.450002) (width 0.25) (layer F.Cu) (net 15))
 (segment (start 160.45 87.450002) (end 160.959999 87.960001) (width 0.25) (layer F.Cu) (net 15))
 (segment (start 161.5 89.15) (end 161.25 89.4) (width 0.25) (layer B.Cu) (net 15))
 (segment (start 161.5 88.500002) (end 161.5 89.15) (width 0.25) (layer B.Cu) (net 15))
 (segment (start 165.75 89.35) (end 164.25 89.35) (width 0.25) (layer B.Cu) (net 14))
 (segment (start 160.959999 81.439999) (end 160.959999 86.334999) (width 0.25) (layer F.Cu) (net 14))
 (segment (start 159.96 80.44) (end 160.959999 81.439999) (width 0.25) (layer F.Cu) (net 14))
 (segment (start 160.959999 86.334999) (end 162.975 88.35) (width 0.25) (layer F.Cu) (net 14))
 (via (at 164.775 88.45) (size 0.6) (drill 0.3) (layers F.Cu B.Cu) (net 14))
 (segment (start 162.975 88.35) (end 164.675 88.35) (width 0.25) (layer F.Cu) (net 14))
 (segment (start 164.675 88.35) (end 164.775 88.45) (width 0.25) (layer F.Cu) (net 14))
 (segment (start 164.775 88.825) (end 164.25 89.35) (width 0.25) (layer B.Cu) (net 14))
 (segment (start 164.775 88.45) (end 164.775 88.825) (width 0.25) (layer B.Cu) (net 14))
 (segment (start 146.25 85.575) (end 146.025 85.35) (width 0.25) (layer B.Cu) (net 8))
 (segment (start 146.25 87.6) (end 146.25 85.575) (width 0.25) (layer B.Cu) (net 8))
 (segment (start 143.485 85.915) (end 143.485 85.35) (width 0.25) (layer B.Cu) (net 9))
 (segment (start 141.75 87.6) (end 141.8 87.6) (width 0.25) (layer B.Cu) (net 9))
 (segment (start 141.8 87.6) (end 143.485 85.915) (width 0.25) (layer B.Cu) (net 9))
 (segment (start 152.75 86.225) (end 151.825 85.3) (width 0.25) (layer B.Cu) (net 6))
 (segment (start 152.75 87.6) (end 152.75 86.225) (width 0.25) (layer B.Cu) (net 6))
 (segment (start 148.25 86.335) (end 149.285 85.3) (width 0.25) (layer B.Cu) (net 7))
 (segment (start 148.25 87.6) (end 148.25 86.335) (width 0.25) (layer B.Cu) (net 7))
 (segment (start 148.325 76.425) (end 143.5 76.425) (width 0.25) (layer F.Cu) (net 12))
 (segment (start 149.8 77.9) (end 148.325 76.425) (width 0.25) (layer F.Cu) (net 12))
 (segment (start 143.5 77.839213) (end 143.5 82.925) (width 0.25) (layer B.Cu) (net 12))
 (segment (start 143.5 76.425) (end 143.5 77.839213) (width 0.25) (layer B.Cu) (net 12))
 (segment (start 159.25 86.325) (end 158.175 85.25) (width 0.25) (layer B.Cu) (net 4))
 (segment (start 159.25 87.6) (end 159.25 86.325) (width 0.25) (layer B.Cu) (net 4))
 (segment (start 154.75 86.135) (end 155.635 85.25) (width 0.25) (layer B.Cu) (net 5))
 (segment (start 154.75 87.6) (end 154.75 86.135) (width 0.25) (layer B.Cu) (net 5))
 (segment (start 165.75 86.625) (end 165.75 87.55) (width 0.25) (layer B.Cu) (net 1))
 (segment (start 164.325 85.2) (end 165.75 86.625) (width 0.25) (layer B.Cu) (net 1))
 (segment (start 161.25 85.735) (end 161.785 85.2) (width 0.25) (layer B.Cu) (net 3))
 (segment (start 161.25 87.6) (end 161.25 85.735) (width 0.25) (layer B.Cu) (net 3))
 (segment (start 166.025 80.95) (end 168.675 80.95) (width 0.25) (layer B.Cu) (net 11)))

